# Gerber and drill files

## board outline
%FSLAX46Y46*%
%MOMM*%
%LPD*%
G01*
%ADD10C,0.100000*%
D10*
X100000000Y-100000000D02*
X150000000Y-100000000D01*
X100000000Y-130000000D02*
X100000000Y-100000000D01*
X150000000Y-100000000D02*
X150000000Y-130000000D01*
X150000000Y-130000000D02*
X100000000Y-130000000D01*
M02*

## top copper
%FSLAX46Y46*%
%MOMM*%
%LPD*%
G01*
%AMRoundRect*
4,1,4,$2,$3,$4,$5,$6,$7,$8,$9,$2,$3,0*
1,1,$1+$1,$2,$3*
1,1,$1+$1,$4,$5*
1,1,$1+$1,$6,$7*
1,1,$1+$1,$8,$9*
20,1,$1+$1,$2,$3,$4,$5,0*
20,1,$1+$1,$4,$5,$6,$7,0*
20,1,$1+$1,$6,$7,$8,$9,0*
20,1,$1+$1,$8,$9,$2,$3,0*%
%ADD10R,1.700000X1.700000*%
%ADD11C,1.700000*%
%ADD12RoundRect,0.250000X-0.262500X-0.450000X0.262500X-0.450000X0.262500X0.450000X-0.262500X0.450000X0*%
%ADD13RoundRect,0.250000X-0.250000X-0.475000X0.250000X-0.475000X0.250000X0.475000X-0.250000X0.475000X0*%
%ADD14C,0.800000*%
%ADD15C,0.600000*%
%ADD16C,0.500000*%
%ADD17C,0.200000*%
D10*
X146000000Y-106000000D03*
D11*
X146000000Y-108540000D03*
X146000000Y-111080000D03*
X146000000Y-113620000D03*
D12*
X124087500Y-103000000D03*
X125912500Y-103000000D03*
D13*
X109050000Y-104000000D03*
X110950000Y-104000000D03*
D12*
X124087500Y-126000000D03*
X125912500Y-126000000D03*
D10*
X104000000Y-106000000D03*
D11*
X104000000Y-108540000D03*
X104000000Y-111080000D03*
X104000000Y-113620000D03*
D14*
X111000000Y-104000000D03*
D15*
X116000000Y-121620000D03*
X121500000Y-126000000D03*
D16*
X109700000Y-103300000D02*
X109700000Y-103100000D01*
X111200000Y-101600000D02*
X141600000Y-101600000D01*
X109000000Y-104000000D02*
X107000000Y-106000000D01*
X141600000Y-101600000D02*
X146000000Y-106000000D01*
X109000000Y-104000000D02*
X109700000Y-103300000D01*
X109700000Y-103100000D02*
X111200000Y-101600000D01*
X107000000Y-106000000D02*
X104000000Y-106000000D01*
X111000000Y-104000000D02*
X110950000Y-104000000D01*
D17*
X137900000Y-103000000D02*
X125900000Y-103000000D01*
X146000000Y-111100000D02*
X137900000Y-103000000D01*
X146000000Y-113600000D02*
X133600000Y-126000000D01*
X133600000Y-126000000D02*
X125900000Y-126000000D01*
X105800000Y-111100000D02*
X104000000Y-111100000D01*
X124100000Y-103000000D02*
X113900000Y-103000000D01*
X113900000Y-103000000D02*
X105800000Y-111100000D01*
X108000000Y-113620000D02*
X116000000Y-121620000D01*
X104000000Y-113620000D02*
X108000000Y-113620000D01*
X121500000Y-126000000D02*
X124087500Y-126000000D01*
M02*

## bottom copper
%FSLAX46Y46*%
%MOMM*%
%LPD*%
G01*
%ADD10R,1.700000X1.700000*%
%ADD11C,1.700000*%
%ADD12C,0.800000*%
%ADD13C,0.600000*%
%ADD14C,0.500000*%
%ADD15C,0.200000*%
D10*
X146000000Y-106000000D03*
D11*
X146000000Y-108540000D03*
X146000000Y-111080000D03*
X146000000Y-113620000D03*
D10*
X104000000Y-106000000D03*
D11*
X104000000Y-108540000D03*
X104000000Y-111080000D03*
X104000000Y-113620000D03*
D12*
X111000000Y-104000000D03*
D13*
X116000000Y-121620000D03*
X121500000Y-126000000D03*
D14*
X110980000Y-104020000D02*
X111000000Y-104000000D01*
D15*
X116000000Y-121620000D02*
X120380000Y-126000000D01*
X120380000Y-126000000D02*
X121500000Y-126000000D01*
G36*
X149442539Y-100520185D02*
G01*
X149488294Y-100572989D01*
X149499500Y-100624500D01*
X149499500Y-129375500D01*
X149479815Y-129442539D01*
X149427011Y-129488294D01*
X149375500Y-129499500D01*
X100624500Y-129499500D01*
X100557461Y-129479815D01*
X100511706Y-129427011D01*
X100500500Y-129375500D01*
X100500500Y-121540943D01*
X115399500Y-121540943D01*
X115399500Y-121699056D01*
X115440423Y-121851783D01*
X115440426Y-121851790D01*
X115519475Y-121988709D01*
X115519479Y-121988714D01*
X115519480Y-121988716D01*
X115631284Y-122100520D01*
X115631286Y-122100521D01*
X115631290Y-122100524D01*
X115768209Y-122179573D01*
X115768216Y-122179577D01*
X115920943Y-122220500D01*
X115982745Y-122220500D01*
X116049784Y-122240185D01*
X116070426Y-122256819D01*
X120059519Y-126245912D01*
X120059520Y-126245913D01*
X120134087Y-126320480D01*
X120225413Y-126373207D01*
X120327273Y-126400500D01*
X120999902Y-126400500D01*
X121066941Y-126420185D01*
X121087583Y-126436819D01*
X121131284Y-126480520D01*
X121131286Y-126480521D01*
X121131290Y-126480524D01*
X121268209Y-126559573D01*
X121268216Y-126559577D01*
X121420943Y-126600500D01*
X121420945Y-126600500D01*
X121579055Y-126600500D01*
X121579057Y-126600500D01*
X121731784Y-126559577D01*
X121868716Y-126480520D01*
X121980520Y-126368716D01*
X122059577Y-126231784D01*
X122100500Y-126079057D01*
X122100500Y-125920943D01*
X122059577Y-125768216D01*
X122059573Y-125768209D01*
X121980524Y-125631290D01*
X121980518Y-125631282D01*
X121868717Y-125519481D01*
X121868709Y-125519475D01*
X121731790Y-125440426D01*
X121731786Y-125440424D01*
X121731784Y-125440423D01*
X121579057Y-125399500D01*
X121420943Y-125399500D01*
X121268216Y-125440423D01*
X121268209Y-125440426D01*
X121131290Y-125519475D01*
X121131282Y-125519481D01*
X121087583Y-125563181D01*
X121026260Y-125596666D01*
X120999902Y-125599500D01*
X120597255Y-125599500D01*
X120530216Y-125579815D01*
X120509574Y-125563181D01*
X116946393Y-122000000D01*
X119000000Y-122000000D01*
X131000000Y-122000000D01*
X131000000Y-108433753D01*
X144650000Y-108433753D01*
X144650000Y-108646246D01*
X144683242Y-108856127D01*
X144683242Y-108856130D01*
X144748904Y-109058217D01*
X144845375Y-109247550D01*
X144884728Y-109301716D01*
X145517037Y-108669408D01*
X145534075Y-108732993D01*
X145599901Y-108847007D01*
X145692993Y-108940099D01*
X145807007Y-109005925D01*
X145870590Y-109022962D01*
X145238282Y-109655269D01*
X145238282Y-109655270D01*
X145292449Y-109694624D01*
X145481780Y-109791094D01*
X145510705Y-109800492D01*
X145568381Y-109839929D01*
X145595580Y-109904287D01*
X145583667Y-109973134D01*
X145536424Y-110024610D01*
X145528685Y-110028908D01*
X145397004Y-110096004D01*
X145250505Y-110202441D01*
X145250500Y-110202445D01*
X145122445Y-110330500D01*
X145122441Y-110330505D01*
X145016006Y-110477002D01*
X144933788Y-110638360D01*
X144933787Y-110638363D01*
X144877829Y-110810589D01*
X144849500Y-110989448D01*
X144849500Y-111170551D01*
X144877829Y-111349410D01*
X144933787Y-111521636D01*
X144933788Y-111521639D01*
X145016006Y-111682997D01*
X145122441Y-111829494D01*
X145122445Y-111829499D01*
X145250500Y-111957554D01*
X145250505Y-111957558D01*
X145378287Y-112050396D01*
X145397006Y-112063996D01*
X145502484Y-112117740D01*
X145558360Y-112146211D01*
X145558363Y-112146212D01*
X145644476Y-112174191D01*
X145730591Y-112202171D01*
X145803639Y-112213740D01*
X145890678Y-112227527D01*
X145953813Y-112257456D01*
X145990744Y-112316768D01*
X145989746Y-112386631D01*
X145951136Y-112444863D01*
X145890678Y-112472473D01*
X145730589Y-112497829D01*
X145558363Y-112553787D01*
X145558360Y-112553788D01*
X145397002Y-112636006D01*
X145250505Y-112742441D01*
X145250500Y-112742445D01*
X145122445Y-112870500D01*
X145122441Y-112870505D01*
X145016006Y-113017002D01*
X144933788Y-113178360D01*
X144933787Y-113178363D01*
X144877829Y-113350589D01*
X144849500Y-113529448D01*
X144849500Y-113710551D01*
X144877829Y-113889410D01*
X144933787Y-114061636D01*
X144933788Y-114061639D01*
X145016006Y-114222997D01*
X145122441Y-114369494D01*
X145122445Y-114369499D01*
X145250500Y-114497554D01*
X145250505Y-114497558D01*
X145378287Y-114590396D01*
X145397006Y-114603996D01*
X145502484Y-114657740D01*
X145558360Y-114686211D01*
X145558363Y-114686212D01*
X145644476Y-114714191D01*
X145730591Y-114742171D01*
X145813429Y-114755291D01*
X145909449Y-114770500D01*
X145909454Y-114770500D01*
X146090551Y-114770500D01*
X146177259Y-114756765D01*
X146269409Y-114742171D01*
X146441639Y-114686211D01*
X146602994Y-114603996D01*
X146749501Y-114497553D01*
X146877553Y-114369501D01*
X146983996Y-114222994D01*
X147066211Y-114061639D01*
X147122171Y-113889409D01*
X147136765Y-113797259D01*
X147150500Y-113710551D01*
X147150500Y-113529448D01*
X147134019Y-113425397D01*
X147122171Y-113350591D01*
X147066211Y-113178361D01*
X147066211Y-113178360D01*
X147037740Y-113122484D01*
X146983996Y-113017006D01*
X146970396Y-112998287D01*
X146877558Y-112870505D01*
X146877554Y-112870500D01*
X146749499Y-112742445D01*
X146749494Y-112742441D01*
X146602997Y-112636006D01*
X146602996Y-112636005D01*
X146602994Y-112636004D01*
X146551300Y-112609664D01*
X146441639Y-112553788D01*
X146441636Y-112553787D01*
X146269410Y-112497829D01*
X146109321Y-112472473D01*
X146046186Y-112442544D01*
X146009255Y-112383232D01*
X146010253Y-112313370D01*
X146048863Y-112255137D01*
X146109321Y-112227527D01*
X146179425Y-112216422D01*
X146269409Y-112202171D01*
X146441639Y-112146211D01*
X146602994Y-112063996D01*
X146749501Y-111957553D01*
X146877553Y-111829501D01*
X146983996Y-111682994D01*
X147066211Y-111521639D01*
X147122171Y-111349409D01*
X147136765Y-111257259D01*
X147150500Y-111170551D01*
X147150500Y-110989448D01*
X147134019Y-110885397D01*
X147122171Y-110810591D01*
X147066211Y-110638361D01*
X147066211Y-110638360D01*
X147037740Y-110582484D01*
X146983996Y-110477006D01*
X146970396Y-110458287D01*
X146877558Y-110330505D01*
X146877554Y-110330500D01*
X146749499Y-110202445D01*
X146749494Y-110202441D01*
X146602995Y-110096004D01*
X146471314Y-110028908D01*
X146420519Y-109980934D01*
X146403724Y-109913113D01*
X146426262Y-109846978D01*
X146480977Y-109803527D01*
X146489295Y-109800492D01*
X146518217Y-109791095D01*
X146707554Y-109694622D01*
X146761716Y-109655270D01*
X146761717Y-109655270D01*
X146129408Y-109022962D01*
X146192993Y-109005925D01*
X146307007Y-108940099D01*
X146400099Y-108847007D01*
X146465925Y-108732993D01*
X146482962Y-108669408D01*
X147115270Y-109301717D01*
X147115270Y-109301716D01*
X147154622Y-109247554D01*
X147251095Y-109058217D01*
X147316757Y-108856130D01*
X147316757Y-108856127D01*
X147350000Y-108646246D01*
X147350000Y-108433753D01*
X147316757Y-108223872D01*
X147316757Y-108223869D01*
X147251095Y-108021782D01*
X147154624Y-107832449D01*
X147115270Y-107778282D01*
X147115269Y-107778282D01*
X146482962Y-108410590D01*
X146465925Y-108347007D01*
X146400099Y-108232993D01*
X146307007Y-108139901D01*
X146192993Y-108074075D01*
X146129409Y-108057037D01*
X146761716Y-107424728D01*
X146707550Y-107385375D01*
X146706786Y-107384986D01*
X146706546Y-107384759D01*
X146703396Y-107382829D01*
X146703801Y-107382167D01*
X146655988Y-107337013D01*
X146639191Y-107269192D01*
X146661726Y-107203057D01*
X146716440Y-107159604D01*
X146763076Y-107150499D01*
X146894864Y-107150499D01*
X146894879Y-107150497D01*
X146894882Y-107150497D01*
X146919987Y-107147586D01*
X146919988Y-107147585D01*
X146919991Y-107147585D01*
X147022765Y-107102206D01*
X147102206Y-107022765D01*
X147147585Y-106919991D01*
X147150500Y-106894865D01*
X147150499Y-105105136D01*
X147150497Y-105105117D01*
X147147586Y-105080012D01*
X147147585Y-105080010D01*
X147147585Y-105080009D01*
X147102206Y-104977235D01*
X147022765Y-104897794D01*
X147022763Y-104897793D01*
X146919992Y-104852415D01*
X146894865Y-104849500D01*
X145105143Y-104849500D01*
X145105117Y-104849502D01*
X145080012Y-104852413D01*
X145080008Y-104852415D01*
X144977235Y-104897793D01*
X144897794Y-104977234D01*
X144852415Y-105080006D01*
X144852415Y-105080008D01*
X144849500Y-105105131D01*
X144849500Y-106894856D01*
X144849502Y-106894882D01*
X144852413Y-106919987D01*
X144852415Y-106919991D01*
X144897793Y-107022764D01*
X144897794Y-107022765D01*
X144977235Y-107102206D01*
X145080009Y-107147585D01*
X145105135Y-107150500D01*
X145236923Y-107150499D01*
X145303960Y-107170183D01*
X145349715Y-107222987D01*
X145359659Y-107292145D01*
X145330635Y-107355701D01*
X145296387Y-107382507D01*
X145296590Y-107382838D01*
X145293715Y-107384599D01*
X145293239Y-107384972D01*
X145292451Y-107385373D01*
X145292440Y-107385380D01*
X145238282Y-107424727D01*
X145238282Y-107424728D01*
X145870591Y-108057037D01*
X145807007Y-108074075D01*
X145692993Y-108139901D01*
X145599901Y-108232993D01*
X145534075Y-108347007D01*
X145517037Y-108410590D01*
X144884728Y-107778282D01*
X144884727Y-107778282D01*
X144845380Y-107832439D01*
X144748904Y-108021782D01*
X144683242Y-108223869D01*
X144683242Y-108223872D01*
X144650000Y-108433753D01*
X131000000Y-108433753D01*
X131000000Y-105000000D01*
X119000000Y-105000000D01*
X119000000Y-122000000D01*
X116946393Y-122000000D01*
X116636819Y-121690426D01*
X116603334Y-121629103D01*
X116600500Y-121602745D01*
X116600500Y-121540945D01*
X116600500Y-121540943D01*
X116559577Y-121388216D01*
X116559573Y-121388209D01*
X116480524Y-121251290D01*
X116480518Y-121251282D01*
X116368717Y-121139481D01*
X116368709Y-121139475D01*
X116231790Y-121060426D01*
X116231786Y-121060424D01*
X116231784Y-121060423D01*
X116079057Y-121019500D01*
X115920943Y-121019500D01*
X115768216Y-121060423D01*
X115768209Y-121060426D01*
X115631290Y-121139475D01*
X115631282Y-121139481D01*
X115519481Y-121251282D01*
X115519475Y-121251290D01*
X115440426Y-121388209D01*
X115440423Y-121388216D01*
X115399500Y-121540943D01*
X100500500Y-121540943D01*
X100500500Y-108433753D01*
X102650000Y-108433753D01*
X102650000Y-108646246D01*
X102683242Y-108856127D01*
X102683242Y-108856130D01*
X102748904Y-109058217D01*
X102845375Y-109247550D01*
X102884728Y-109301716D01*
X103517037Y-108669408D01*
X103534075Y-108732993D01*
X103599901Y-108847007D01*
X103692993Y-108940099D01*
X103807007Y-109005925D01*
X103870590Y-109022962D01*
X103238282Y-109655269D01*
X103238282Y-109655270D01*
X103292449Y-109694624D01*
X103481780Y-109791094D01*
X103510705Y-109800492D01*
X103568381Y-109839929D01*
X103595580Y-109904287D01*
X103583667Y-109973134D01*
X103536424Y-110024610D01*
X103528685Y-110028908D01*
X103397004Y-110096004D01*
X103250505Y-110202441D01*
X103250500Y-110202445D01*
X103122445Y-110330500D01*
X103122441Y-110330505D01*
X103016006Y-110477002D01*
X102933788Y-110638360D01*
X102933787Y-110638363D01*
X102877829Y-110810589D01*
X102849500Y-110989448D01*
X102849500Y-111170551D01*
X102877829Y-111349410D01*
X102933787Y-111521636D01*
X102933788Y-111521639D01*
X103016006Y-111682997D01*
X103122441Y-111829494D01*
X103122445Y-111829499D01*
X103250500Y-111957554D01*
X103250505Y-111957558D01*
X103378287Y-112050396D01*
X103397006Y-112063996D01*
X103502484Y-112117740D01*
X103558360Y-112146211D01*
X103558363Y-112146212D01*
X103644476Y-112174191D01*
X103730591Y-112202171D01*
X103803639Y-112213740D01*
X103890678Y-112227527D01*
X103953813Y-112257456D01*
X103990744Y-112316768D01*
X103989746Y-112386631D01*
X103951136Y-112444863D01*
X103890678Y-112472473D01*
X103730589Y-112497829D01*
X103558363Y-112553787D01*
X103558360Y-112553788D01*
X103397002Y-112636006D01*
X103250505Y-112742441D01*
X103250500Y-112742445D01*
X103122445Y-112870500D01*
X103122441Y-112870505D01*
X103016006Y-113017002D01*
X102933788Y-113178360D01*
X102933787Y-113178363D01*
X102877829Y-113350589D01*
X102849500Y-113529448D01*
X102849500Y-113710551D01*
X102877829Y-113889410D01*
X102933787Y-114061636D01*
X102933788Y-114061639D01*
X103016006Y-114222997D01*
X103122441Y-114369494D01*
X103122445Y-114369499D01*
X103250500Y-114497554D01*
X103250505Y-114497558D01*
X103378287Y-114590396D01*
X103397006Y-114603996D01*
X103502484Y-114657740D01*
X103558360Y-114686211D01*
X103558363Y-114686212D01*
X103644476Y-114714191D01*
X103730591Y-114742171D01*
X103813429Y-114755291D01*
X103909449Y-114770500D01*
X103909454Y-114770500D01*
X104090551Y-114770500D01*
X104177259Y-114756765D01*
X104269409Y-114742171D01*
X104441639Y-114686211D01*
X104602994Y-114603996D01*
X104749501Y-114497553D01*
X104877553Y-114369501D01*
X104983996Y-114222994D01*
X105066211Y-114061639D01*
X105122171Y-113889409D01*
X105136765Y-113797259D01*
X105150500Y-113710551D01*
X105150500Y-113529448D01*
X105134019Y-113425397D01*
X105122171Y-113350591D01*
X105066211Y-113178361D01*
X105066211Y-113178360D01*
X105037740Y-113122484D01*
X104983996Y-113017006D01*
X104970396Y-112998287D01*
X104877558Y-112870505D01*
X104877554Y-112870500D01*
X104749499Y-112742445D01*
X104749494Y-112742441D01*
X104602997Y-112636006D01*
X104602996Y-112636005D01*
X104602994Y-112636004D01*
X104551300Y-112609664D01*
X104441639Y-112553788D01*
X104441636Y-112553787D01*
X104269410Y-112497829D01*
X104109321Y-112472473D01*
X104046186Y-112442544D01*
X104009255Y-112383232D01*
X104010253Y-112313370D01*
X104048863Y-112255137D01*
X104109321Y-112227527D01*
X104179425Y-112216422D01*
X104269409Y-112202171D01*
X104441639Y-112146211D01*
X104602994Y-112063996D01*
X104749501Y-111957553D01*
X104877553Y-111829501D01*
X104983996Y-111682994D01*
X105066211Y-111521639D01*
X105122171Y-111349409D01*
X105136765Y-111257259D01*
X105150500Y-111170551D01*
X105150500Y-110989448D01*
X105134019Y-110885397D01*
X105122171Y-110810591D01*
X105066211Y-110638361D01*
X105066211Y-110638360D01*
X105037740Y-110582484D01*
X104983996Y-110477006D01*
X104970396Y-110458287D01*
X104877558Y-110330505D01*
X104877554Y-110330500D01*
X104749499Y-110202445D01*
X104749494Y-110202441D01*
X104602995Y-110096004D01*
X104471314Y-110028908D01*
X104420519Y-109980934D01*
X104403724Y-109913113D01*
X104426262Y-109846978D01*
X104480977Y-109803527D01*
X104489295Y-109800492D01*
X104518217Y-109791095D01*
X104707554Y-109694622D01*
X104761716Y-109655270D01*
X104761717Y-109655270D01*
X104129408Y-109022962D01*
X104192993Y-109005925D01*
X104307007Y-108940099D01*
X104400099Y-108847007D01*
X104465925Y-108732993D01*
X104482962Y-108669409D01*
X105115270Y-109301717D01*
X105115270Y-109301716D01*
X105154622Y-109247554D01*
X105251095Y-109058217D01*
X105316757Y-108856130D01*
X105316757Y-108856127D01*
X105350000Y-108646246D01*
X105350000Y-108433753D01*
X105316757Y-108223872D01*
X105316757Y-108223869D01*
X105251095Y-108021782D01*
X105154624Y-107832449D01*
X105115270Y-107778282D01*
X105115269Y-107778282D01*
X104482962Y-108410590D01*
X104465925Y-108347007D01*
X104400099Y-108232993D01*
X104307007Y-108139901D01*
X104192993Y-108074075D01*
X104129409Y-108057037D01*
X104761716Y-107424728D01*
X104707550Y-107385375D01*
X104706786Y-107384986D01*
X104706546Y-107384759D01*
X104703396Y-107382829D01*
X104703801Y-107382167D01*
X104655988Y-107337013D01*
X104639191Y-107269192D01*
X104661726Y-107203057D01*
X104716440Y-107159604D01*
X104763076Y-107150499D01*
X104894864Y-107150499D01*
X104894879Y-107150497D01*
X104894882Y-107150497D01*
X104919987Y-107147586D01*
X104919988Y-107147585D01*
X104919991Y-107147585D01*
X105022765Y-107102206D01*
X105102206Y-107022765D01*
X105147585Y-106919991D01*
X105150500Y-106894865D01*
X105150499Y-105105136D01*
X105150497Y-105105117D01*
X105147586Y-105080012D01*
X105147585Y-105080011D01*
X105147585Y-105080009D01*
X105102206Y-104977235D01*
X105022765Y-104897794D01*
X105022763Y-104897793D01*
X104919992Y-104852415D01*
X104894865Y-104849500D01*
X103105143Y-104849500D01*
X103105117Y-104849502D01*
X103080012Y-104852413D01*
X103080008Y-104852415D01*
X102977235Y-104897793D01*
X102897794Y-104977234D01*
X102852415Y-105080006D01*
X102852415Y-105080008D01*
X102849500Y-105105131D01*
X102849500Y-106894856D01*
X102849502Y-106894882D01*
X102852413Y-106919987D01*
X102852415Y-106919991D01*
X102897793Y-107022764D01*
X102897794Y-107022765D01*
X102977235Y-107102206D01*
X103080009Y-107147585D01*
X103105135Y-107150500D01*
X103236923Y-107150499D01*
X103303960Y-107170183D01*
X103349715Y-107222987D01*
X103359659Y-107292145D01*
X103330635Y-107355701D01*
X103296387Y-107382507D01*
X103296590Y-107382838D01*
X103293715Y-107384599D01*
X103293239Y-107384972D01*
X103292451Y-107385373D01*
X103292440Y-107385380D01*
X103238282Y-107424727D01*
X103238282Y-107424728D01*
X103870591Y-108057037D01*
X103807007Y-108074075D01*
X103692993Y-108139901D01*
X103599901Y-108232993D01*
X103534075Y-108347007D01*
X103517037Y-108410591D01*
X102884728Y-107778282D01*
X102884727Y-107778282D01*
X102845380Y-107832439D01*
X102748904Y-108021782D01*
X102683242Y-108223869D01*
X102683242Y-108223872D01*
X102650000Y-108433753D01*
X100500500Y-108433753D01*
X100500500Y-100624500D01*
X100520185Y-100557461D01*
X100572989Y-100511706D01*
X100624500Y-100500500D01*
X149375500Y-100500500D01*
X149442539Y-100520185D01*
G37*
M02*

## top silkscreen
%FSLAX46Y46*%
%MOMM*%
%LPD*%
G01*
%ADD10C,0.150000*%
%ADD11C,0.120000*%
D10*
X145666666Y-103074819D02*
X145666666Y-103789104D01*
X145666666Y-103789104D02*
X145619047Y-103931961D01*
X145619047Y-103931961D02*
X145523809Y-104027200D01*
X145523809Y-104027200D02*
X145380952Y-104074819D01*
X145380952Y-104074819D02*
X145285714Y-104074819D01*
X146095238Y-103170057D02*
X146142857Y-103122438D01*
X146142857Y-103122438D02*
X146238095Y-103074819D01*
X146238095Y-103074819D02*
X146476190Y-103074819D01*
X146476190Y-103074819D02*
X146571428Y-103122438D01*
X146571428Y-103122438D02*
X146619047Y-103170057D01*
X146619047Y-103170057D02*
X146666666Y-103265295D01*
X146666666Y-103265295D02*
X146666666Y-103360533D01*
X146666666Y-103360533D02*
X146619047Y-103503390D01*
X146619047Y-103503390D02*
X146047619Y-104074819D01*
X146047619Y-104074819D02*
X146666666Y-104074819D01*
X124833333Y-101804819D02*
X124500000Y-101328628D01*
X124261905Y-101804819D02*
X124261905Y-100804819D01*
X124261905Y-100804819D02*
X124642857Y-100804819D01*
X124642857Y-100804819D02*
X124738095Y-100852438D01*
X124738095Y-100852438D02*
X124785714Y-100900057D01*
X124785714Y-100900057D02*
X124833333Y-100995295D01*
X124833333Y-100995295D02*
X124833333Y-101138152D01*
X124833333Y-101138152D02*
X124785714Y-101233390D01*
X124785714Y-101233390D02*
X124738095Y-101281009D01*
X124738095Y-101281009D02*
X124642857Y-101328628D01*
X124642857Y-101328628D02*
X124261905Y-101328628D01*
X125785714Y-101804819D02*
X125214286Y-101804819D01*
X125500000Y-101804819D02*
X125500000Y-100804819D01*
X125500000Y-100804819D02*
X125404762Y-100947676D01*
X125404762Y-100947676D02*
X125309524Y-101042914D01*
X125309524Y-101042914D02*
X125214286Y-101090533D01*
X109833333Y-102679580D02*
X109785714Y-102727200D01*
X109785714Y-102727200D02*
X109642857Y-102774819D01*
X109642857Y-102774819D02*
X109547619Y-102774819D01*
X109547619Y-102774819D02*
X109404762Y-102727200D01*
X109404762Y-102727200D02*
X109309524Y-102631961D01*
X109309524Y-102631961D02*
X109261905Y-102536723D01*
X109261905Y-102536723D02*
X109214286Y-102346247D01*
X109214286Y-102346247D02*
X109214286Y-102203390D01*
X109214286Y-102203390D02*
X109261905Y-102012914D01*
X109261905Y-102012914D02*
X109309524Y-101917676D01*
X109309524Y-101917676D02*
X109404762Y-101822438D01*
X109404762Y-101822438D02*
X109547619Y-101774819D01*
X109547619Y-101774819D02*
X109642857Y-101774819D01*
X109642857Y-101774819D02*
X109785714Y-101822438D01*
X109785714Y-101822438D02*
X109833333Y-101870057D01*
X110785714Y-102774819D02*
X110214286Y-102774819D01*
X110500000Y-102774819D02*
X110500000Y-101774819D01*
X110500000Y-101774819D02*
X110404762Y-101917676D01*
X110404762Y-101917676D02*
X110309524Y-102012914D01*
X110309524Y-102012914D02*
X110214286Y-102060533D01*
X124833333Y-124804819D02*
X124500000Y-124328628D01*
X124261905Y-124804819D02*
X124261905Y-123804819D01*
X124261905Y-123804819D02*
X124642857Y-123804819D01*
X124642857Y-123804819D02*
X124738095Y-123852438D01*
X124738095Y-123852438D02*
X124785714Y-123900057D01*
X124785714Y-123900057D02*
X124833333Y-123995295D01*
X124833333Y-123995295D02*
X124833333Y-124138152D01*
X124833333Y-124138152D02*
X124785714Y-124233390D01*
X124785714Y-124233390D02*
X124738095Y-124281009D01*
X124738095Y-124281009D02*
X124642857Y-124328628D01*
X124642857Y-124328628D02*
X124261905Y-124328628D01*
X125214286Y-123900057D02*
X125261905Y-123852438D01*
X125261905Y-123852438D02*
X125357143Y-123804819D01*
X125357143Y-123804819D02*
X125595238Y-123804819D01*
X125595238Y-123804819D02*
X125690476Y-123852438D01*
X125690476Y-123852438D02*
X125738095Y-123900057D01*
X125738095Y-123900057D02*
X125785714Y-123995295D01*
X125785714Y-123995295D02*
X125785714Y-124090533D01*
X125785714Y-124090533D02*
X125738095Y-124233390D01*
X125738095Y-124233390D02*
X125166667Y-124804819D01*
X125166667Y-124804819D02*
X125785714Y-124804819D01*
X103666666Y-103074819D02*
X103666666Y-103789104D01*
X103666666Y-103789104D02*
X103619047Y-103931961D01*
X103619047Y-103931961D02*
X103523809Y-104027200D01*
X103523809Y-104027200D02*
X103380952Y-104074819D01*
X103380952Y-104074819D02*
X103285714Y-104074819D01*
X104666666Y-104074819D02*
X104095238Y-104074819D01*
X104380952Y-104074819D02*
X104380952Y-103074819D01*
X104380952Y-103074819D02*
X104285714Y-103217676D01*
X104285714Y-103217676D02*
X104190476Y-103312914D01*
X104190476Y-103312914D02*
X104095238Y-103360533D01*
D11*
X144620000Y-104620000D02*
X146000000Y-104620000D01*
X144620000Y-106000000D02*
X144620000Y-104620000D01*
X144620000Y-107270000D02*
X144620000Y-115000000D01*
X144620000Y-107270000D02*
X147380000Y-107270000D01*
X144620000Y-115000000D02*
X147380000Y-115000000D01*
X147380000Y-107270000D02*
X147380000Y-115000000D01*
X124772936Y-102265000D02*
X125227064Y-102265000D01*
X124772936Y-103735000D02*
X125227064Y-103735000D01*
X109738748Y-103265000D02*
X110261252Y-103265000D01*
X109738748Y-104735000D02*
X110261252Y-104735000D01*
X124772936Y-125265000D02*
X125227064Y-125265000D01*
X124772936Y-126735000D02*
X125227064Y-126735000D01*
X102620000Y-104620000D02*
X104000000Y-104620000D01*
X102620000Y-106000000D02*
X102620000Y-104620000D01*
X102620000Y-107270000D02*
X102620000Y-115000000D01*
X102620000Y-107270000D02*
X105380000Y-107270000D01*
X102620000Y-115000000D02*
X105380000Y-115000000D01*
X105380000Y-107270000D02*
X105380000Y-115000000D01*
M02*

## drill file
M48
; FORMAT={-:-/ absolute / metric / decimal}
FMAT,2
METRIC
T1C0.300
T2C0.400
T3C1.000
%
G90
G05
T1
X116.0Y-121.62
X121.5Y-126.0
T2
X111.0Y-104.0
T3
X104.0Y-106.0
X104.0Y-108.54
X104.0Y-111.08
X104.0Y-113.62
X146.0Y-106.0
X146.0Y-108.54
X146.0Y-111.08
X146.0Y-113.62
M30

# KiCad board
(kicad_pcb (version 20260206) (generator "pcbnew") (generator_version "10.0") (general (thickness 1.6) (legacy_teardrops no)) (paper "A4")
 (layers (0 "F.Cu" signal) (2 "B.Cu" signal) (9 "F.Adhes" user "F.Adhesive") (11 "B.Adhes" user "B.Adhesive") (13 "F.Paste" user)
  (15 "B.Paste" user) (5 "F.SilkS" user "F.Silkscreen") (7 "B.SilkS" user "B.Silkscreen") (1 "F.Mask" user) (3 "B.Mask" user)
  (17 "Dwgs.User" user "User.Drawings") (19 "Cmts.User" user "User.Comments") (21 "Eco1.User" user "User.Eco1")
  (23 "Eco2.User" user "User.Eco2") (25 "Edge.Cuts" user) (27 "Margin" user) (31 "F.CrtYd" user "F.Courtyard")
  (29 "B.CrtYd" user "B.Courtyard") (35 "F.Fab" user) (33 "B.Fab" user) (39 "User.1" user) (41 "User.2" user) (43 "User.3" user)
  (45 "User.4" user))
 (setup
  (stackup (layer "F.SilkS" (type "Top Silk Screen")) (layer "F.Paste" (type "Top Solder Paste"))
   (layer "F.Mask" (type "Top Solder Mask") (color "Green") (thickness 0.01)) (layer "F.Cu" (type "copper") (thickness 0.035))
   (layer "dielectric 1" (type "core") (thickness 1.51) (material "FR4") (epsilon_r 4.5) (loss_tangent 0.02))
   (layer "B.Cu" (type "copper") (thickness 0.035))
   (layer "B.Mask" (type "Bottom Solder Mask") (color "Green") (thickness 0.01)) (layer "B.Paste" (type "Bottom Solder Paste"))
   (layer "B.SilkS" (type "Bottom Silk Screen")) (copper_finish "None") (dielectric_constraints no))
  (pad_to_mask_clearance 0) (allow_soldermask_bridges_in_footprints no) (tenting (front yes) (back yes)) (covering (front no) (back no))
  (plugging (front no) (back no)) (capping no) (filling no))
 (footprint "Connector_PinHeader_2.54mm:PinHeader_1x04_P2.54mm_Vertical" (layer "F.Cu") (at 146 106)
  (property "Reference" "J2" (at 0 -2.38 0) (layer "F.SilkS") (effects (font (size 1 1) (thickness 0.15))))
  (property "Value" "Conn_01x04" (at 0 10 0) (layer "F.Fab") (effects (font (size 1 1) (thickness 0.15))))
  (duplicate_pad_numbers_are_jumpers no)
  (fp_line (start -1.38 -1.38) (end 0 -1.38) (stroke (width 0.12) (type solid)) (layer "F.SilkS"))
  (fp_line (start -1.38 0) (end -1.38 -1.38) (stroke (width 0.12) (type solid)) (layer "F.SilkS"))
  (fp_line (start -1.38 1.27) (end -1.38 9) (stroke (width 0.12) (type solid)) (layer "F.SilkS"))
  (fp_line (start -1.38 1.27) (end 1.38 1.27) (stroke (width 0.12) (type solid)) (layer "F.SilkS"))
  (fp_line (start -1.38 9) (end 1.38 9) (stroke (width 0.12) (type solid)) (layer "F.SilkS"))
  (fp_line (start 1.38 1.27) (end 1.38 9) (stroke (width 0.12) (type solid)) (layer "F.SilkS"))
  (pad "1" thru_hole rect (at 0 0) (size 1.7 1.7) (drill 1) (layers "*.Cu" "*.Mask") (remove_unused_layers no) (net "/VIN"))
  (pad "2" thru_hole circle (at 0 2.54) (size 1.7 1.7) (drill 1) (layers "*.Cu" "*.Mask") (remove_unused_layers no) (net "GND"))
  (pad "3" thru_hole circle (at 0 5.08) (size 1.7 1.7) (drill 1) (layers "*.Cu" "*.Mask") (remove_unused_layers no) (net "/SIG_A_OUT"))
  (pad "4" thru_hole circle (at 0 7.62) (size 1.7 1.7) (drill 1) (layers "*.Cu" "*.Mask") (remove_unused_layers no) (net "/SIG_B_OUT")))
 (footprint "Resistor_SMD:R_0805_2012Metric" (layer "F.Cu") (at 125 103)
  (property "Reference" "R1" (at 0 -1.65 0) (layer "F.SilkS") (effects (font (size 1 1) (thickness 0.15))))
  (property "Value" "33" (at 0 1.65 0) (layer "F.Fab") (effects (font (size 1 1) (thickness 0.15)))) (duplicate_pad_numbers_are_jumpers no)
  (fp_line (start -0.227064 -0.735) (end 0.227064 -0.735) (stroke (width 0.12) (type solid)) (layer "F.SilkS"))
  (fp_line (start -0.227064 0.735) (end 0.227064 0.735) (stroke (width 0.12) (type solid)) (layer "F.SilkS"))
  (pad "1" smd roundrect (at -0.9125 0) (size 1.025 1.4) (layers "F.Cu" "F.Mask" "F.Paste") (roundrect_rratio 0.243902) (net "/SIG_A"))
  (pad "2" smd roundrect (at 0.9125 0) (size 1.025 1.4) (layers "F.Cu" "F.Mask" "F.Paste") (roundrect_rratio 0.243902) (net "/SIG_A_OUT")))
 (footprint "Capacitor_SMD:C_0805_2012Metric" (layer "F.Cu") (at 110 104)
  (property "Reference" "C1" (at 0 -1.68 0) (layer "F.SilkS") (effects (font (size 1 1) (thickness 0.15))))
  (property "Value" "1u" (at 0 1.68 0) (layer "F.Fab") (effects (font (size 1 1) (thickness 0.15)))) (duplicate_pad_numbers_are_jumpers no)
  (fp_line (start -0.261252 -0.735) (end 0.261252 -0.735) (stroke (width 0.12) (type solid)) (layer "F.SilkS"))
  (fp_line (start -0.261252 0.735) (end 0.261252 0.735) (stroke (width 0.12) (type solid)) (layer "F.SilkS"))
  (pad "1" smd roundrect (at -0.95 0) (size 1 1.45) (layers "F.Cu" "F.Mask" "F.Paste") (roundrect_rratio 0.25) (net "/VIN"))
  (pad "2" smd roundrect (at 0.95 0) (size 1 1.45) (layers "F.Cu" "F.Mask" "F.Paste") (roundrect_rratio 0.25) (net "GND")))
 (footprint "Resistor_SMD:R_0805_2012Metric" (layer "F.Cu") (at 125 126)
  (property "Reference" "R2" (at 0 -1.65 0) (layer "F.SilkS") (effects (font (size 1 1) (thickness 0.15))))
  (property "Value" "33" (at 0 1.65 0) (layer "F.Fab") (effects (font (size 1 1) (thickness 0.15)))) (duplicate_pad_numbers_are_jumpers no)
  (fp_line (start -0.227064 -0.735) (end 0.227064 -0.735) (stroke (width 0.12) (type solid)) (layer "F.SilkS"))
  (fp_line (start -0.227064 0.735) (end 0.227064 0.735) (stroke (width 0.12) (type solid)) (layer "F.SilkS"))
  (pad "1" smd roundrect (at -0.9125 0) (size 1.025 1.4) (layers "F.Cu" "F.Mask" "F.Paste") (roundrect_rratio 0.243902) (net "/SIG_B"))
  (pad "2" smd roundrect (at 0.9125 0) (size 1.025 1.4) (layers "F.Cu" "F.Mask" "F.Paste") (roundrect_rratio 0.243902) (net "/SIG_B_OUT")))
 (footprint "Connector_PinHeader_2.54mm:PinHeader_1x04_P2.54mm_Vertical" (layer "F.Cu") (at 104 106)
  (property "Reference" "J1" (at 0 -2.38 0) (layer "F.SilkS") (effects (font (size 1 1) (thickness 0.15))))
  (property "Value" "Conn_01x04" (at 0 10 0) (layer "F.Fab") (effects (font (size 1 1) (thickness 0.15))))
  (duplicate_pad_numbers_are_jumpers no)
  (fp_line (start -1.38 -1.38) (end 0 -1.38) (stroke (width 0.12) (type solid)) (layer "F.SilkS"))
  (fp_line (start -1.38 0) (end -1.38 -1.38) (stroke (width 0.12) (type solid)) (layer "F.SilkS"))
  (fp_line (start -1.38 1.27) (end -1.38 9) (stroke (width 0.12) (type solid)) (layer "F.SilkS"))
  (fp_line (start -1.38 1.27) (end 1.38 1.27) (stroke (width 0.12) (type solid)) (layer "F.SilkS"))
  (fp_line (start -1.38 9) (end 1.38 9) (stroke (width 0.12) (type solid)) (layer "F.SilkS"))
  (fp_line (start 1.38 1.27) (end 1.38 9) (stroke (width 0.12) (type solid)) (layer "F.SilkS"))
  (pad "1" thru_hole rect (at 0 0) (size 1.7 1.7) (drill 1) (layers "*.Cu" "*.Mask") (remove_unused_layers no) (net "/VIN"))
  (pad "2" thru_hole circle (at 0 2.54) (size 1.7 1.7) (drill 1) (layers "*.Cu" "*.Mask") (remove_unused_layers no) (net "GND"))
  (pad "3" thru_hole circle (at 0 5.08) (size 1.7 1.7) (drill 1) (layers "*.Cu" "*.Mask") (remove_unused_layers no) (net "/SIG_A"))
  (pad "4" thru_hole circle (at 0 7.62) (size 1.7 1.7) (drill 1) (layers "*.Cu" "*.Mask") (remove_unused_layers no) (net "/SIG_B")))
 (gr_line (start 100 100) (end 150 100) (stroke (width 0.1) (type default)) (layer "Edge.Cuts"))
 (gr_line (start 100 130) (end 100 100) (stroke (width 0.1) (type default)) (layer "Edge.Cuts"))
 (gr_line (start 150 100) (end 150 130) (stroke (width 0.1) (type default)) (layer "Edge.Cuts"))
 (gr_line (start 150 130) (end 100 130) (stroke (width 0.1) (type default)) (layer "Edge.Cuts"))
 (segment (start 109.7 103.3) (end 109.7 103.1) (width 0.5) (layer "F.Cu") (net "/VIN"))
 (segment (start 111.2 101.6) (end 141.6 101.6) (width 0.5) (layer "F.Cu") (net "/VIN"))
 (segment (start 109 104) (end 107 106) (width 0.5) (layer "F.Cu") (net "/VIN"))
 (segment (start 141.6 101.6) (end 146 106) (width 0.5) (layer "F.Cu") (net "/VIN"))
 (segment (start 109 104) (end 109.7 103.3) (width 0.5) (layer "F.Cu") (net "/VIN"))
 (segment (start 109.7 103.1) (end 111.2 101.6) (width 0.5) (layer "F.Cu") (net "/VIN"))
 (segment (start 107 106) (end 104 106) (width 0.5) (layer "F.Cu") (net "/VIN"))
 (segment (start 111 104) (end 110.95 104) (width 0.5) (layer "F.Cu") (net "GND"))
 (via (at 111 104) (size 0.8) (drill 0.4) (layers "F.Cu" "B.Cu") (capping yes) (filling yes) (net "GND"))
 (segment (start 110.98 104.02) (end 111 104) (width 0.5) (layer "B.Cu") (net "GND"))
 (segment (start 137.9 103) (end 125.9 103) (width 0.2) (layer "F.Cu") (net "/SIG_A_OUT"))
 (segment (start 146 111.1) (end 137.9 103) (width 0.2) (layer "F.Cu") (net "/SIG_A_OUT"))
 (segment (start 146 113.6) (end 133.6 126) (width 0.2) (layer "F.Cu") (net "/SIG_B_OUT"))
 (segment (start 133.6 126) (end 125.9 126) (width 0.2) (layer "F.Cu") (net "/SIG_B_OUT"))
 (segment (start 105.8 111.1) (end 104 111.1) (width 0.2) (layer "F.Cu") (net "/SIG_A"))
 (segment (start 124.1 103) (end 113.9 103) (width 0.2) (layer "F.Cu") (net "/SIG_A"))
 (segment (start 113.9 103) (end 105.8 111.1) (width 0.2) (layer "F.Cu") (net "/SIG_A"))
 (segment (start 108 113.62) (end 116 121.62) (width 0.2) (locked yes) (layer "F.Cu") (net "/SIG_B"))
 (segment (start 104 113.62) (end 108 113.62) (width 0.2) (locked yes) (layer "F.Cu") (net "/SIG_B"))
 (segment (start 121.5 126) (end 124.0875 126) (width 0.2) (locked yes) (layer "F.Cu") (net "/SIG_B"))
 (via (at 116 121.62) (size 0.6) (drill 0.3) (layers "F.Cu" "B.Cu") (locked yes) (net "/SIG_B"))
 (via (at 121.5 126) (size 0.6) (drill 0.3) (layers "F.Cu" "B.Cu") (locked yes) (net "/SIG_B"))
 (segment (start 116 121.62) (end 120.38 126) (width 0.2) (locked yes) (layer "B.Cu") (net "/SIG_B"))
 (segment (start 120.38 126) (end 121.5 126) (width 0.2) (locked yes) (layer "B.Cu") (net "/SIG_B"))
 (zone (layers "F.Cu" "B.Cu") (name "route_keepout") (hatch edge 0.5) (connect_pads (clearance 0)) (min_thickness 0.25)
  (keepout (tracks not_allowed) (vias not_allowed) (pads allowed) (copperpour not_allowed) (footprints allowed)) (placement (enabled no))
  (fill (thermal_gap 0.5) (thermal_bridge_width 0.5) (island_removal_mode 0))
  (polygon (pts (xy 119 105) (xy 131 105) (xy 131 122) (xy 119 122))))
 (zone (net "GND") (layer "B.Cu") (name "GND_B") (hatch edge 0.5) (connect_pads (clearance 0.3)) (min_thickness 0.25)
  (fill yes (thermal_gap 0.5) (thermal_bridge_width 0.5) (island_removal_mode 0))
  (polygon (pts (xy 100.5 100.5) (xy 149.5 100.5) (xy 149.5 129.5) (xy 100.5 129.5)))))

